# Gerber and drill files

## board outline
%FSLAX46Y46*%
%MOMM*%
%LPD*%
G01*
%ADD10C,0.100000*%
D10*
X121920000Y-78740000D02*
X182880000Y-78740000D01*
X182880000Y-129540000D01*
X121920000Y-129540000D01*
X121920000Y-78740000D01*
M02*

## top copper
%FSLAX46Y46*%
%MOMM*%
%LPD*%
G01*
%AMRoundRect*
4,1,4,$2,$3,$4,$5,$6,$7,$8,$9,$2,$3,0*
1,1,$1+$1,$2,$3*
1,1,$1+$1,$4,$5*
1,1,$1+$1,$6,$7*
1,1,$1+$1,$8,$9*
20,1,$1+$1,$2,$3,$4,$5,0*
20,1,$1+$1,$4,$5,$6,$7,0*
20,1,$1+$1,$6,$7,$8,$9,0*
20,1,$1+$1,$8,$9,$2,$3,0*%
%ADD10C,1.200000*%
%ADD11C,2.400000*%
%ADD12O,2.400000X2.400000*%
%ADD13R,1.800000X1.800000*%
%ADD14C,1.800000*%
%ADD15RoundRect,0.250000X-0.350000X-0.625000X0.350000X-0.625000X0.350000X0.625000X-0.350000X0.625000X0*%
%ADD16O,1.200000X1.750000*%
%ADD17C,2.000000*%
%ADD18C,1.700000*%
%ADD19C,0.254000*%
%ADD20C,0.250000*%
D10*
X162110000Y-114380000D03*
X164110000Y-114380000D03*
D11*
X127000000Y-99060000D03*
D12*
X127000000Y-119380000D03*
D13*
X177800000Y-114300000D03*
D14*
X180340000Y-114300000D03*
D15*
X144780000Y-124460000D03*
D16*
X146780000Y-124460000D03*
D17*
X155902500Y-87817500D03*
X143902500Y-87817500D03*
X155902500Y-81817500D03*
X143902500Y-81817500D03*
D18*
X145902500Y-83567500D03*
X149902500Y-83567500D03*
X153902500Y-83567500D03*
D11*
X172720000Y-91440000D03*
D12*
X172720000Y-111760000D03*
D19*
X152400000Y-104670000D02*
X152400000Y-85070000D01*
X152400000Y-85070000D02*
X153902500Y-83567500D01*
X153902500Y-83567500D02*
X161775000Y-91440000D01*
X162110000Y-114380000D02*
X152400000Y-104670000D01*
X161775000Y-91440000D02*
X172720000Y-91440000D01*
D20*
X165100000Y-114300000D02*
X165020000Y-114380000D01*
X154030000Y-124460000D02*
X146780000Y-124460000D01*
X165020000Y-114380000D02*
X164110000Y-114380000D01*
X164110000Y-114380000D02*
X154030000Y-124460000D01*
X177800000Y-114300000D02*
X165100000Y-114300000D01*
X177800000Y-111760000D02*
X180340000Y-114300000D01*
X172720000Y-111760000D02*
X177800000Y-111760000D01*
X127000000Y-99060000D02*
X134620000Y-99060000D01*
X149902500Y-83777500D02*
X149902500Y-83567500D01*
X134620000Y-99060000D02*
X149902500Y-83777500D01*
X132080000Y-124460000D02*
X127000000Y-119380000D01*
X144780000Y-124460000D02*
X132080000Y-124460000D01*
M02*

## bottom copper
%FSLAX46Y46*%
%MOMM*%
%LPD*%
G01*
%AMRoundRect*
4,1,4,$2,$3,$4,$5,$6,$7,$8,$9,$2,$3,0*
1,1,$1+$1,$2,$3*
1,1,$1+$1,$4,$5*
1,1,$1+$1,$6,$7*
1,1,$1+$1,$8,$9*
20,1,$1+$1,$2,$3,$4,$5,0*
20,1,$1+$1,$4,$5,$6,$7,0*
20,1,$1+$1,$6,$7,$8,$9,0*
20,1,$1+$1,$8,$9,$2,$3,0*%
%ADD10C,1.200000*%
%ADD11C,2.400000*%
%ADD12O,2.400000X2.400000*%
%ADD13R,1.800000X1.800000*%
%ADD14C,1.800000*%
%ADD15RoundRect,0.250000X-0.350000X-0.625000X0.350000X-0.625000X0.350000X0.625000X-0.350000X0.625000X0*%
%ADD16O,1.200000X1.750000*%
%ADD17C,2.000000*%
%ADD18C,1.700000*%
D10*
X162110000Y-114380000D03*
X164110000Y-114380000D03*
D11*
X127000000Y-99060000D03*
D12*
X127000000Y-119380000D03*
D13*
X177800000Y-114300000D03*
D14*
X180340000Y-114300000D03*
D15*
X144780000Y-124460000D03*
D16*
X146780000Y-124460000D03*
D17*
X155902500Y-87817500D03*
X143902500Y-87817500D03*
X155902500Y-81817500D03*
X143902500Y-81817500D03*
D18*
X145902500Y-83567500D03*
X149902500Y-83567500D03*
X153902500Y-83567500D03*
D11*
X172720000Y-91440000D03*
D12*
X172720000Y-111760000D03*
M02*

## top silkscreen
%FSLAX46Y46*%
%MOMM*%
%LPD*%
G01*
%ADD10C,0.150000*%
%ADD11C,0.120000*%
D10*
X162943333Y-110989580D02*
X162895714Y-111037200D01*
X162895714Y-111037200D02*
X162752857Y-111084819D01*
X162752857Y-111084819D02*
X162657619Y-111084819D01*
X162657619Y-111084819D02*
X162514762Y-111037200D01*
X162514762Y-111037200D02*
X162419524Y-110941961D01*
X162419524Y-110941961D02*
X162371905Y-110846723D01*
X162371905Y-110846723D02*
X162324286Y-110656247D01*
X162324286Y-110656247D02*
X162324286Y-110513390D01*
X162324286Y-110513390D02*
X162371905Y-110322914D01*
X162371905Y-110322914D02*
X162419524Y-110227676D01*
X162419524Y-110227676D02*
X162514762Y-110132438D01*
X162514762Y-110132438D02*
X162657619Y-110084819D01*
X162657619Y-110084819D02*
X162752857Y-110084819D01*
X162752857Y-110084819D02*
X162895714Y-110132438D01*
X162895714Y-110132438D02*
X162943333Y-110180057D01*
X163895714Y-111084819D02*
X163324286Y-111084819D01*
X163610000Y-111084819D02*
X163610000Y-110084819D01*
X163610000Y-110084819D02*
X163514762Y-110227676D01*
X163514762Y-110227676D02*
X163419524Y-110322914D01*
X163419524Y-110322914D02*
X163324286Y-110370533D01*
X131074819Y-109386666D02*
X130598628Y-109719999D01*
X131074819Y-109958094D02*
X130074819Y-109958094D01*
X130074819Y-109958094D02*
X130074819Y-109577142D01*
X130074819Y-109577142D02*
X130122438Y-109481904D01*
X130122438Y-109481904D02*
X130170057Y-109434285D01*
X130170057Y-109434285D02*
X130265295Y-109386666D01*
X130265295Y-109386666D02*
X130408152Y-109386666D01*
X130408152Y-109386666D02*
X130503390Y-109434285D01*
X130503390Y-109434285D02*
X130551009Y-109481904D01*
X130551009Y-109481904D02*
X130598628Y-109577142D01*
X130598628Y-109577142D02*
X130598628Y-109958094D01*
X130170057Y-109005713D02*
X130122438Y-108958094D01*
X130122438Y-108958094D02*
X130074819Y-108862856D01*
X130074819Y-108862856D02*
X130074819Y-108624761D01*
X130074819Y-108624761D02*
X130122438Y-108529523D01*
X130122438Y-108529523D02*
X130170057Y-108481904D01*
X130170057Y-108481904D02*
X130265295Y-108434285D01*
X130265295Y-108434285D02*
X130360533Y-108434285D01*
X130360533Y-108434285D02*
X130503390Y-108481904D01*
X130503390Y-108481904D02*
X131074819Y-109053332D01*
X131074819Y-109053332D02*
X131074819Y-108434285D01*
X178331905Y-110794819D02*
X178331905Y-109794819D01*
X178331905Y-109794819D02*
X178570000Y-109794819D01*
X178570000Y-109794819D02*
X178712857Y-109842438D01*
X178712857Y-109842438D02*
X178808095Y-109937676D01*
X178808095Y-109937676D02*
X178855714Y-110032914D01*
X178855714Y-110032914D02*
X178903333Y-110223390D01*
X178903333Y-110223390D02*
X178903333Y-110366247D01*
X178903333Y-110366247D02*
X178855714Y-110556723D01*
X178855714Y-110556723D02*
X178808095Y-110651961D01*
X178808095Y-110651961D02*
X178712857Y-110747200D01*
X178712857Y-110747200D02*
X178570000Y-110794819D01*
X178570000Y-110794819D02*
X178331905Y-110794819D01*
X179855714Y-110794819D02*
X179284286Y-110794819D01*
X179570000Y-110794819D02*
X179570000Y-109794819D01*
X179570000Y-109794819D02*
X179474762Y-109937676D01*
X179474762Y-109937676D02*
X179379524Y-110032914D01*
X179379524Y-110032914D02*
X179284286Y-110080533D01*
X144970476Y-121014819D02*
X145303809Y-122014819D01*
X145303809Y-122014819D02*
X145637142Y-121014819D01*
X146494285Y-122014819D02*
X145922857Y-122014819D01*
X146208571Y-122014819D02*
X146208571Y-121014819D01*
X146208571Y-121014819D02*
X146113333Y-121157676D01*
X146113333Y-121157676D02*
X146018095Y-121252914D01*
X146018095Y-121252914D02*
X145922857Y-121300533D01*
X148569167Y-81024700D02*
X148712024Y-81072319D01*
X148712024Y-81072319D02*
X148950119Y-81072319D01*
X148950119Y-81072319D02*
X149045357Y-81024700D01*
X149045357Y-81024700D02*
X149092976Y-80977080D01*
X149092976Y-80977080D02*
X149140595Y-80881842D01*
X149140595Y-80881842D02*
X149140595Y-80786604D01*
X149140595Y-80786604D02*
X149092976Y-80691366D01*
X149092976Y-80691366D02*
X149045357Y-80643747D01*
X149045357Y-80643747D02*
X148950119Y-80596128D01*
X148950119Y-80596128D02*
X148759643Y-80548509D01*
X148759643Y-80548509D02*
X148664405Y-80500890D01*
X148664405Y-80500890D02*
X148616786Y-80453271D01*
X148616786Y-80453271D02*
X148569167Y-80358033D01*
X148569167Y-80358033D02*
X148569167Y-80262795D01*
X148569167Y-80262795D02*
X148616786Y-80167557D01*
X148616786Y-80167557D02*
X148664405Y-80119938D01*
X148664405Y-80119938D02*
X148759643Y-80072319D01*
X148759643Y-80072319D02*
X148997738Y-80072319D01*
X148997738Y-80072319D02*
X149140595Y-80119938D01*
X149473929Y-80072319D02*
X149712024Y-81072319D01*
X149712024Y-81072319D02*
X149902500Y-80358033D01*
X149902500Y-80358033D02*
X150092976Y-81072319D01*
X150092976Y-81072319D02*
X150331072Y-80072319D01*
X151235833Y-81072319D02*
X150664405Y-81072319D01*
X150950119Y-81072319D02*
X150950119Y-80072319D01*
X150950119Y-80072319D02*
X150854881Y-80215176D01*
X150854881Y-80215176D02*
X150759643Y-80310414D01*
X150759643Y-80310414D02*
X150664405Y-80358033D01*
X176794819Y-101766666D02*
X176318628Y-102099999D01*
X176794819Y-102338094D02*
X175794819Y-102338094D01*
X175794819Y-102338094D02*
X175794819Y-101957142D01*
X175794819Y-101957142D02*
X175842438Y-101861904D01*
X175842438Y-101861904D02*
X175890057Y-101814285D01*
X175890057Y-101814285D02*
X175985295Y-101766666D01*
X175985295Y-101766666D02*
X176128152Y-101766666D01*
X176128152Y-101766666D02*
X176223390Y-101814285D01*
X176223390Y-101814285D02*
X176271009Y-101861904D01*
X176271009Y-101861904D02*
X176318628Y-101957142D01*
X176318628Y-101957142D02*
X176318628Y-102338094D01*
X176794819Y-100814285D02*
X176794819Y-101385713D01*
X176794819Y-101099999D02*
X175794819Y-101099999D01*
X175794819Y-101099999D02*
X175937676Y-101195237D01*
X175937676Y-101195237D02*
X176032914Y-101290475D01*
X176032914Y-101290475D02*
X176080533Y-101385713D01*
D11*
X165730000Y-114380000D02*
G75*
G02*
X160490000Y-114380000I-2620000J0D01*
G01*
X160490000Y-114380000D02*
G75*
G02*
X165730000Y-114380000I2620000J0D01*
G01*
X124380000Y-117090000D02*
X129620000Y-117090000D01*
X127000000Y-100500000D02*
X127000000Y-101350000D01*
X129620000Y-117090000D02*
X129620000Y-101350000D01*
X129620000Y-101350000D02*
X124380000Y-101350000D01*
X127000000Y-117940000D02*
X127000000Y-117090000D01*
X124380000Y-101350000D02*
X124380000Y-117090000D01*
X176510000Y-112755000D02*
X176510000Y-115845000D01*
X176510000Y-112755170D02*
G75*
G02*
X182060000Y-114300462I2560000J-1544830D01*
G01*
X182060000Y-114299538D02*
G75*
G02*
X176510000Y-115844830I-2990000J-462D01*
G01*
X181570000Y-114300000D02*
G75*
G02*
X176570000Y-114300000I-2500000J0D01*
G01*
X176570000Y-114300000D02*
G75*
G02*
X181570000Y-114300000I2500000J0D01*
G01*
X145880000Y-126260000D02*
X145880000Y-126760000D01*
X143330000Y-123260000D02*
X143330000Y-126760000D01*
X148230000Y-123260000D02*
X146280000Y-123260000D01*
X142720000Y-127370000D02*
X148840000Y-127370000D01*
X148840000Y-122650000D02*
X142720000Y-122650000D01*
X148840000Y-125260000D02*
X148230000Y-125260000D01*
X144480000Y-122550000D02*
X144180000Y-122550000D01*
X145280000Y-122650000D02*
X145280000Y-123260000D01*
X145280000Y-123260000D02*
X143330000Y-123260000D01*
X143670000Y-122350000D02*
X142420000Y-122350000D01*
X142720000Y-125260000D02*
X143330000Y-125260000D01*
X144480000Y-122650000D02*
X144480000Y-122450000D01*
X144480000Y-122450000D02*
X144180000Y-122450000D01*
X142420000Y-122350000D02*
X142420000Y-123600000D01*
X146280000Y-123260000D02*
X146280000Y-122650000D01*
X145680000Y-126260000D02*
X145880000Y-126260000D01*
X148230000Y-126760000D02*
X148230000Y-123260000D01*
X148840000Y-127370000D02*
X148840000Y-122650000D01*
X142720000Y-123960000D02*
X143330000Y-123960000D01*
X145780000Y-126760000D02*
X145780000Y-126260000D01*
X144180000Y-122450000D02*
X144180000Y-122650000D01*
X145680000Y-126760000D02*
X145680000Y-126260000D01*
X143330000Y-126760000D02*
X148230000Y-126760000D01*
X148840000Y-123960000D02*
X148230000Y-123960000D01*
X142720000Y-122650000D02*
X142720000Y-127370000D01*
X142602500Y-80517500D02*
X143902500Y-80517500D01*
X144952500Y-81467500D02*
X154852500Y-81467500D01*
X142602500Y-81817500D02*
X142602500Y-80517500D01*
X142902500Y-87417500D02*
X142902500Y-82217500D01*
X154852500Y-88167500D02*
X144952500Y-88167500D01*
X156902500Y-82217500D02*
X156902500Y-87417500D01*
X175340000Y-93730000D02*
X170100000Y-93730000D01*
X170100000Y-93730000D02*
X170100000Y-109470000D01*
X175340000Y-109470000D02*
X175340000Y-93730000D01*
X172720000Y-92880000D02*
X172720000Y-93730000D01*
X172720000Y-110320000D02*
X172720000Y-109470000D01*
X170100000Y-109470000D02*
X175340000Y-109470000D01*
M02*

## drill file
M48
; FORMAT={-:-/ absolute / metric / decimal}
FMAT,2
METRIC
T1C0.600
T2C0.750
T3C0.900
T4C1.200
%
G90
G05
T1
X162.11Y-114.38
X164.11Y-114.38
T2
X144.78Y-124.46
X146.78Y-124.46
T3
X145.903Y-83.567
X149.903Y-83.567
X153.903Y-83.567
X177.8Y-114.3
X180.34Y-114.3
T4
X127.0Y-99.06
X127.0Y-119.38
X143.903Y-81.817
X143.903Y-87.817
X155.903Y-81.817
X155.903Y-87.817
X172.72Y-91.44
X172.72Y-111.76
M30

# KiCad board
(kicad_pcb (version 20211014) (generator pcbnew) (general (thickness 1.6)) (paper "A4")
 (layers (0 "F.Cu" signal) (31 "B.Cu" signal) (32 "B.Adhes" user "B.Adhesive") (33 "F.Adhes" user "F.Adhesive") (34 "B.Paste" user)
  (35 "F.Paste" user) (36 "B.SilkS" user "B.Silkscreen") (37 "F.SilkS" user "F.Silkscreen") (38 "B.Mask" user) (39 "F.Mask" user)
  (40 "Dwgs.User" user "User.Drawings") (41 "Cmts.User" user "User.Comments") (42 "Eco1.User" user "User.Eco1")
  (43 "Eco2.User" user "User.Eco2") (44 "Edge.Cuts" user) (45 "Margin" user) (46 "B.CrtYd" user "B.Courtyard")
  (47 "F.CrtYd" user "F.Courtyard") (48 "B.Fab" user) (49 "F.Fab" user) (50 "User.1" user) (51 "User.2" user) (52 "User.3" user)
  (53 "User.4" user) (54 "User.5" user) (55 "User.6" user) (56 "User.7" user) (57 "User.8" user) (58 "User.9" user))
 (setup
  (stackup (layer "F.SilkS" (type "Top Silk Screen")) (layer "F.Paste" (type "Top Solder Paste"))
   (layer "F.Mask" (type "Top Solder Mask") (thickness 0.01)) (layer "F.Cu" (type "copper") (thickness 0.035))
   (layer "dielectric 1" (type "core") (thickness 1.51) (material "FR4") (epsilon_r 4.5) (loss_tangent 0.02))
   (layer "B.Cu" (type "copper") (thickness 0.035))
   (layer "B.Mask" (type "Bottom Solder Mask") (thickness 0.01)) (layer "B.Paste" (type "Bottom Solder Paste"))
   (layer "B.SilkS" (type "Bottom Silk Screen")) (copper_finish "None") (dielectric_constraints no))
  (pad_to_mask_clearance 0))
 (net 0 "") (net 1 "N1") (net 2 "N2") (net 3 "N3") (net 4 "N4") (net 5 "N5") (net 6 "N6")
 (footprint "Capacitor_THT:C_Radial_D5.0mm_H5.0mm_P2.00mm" (layer "F.Cu") (at 162.11 114.38)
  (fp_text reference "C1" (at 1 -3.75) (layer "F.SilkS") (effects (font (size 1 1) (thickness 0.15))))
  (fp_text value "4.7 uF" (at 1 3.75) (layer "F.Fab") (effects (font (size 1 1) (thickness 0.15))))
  (fp_circle (center 1 0) (end 3.62 0) (layer "F.SilkS") (width 0.12) (fill none))
  (pad "1" thru_hole circle (at 0 0) (size 1.2 1.2) (drill 0.6) (layers *.Cu *.Mask) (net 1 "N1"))
  (pad "2" thru_hole circle (at 2 0) (size 1.2 1.2) (drill 0.6) (layers *.Cu *.Mask) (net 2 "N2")))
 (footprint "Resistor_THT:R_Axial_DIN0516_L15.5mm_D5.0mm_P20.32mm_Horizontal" (layer "F.Cu") (at 127 99.06 -90)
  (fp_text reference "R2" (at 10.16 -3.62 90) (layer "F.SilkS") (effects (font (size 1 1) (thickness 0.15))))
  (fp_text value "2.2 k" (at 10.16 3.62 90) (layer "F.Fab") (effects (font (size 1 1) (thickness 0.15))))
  (fp_line (start 18.03 2.62) (end 18.03 -2.62) (layer "F.SilkS") (width 0.12))
  (fp_line (start 1.44 0) (end 2.29 0) (layer "F.SilkS") (width 0.12))
  (fp_line (start 18.03 -2.62) (end 2.29 -2.62) (layer "F.SilkS") (width 0.12))
  (fp_line (start 2.29 -2.62) (end 2.29 2.62) (layer "F.SilkS") (width 0.12))
  (fp_line (start 18.88 0) (end 18.03 0) (layer "F.SilkS") (width 0.12))
  (fp_line (start 2.29 2.62) (end 18.03 2.62) (layer "F.SilkS") (width 0.12))
  (pad "1" thru_hole circle (at 0 0 270) (size 2.4 2.4) (drill 1.2) (layers *.Cu *.Mask) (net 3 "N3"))
  (pad "2" thru_hole oval (at 20.32 0 270) (size 2.4 2.4) (drill 1.2) (layers *.Cu *.Mask) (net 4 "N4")))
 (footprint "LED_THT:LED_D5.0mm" (layer "F.Cu") (at 177.8 114.3)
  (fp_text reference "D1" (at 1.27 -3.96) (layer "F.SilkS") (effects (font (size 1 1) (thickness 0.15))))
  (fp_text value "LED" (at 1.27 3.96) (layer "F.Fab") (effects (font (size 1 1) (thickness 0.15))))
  (fp_line (start -1.29 -1.545) (end -1.29 1.545) (layer "F.SilkS") (width 0.12))
  (fp_arc (start -1.29 -1.54483) (mid 2.072002 -2.880433) (end 4.26 0.000462) (layer "F.SilkS") (width 0.12))
  (fp_arc (start 4.26 -0.000462) (mid 2.072002 2.880433) (end -1.29 1.54483) (layer "F.SilkS") (width 0.12))
  (fp_circle (center 1.27 0) (end 3.77 0) (layer "F.SilkS") (width 0.12) (fill none))
  (pad "1" thru_hole rect (at 0 0) (size 1.8 1.8) (drill 0.9) (layers *.Cu *.Mask) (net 2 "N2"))
  (pad "2" thru_hole circle (at 2.54 0) (size 1.8 1.8) (drill 0.9) (layers *.Cu *.Mask) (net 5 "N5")))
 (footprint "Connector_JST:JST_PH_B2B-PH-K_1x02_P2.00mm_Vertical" (layer "F.Cu") (at 144.78 124.46)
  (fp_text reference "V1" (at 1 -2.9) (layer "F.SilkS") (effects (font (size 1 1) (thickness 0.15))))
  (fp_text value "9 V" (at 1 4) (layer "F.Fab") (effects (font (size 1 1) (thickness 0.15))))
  (fp_line (start 1.1 1.8) (end 1.1 2.3) (layer "F.SilkS") (width 0.12))
  (fp_line (start -1.45 -1.2) (end -1.45 2.3) (layer "F.SilkS") (width 0.12))
  (fp_line (start 3.45 -1.2) (end 1.5 -1.2) (layer "F.SilkS") (width 0.12))
  (fp_line (start -2.06 2.91) (end 4.06 2.91) (layer "F.SilkS") (width 0.12))
  (fp_line (start 4.06 -1.81) (end -2.06 -1.81) (layer "F.SilkS") (width 0.12))
  (fp_line (start 4.06 0.8) (end 3.45 0.8) (layer "F.SilkS") (width 0.12))
  (fp_line (start -0.3 -1.91) (end -0.6 -1.91) (layer "F.SilkS") (width 0.12))
  (fp_line (start 0.5 -1.81) (end 0.5 -1.2) (layer "F.SilkS") (width 0.12))
  (fp_line (start 0.5 -1.2) (end -1.45 -1.2) (layer "F.SilkS") (width 0.12))
  (fp_line (start -1.11 -2.11) (end -2.36 -2.11) (layer "F.SilkS") (width 0.12))
  (fp_line (start -2.06 0.8) (end -1.45 0.8) (layer "F.SilkS") (width 0.12))
  (fp_line (start -0.3 -1.81) (end -0.3 -2.01) (layer "F.SilkS") (width 0.12))
  (fp_line (start -0.3 -2.01) (end -0.6 -2.01) (layer "F.SilkS") (width 0.12))
  (fp_line (start -2.36 -2.11) (end -2.36 -0.86) (layer "F.SilkS") (width 0.12))
  (fp_line (start 1.5 -1.2) (end 1.5 -1.81) (layer "F.SilkS") (width 0.12))
  (fp_line (start 0.9 1.8) (end 1.1 1.8) (layer "F.SilkS") (width 0.12))
  (fp_line (start 3.45 2.3) (end 3.45 -1.2) (layer "F.SilkS") (width 0.12))
  (fp_line (start 4.06 2.91) (end 4.06 -1.81) (layer "F.SilkS") (width 0.12))
  (fp_line (start -2.06 -0.5) (end -1.45 -0.5) (layer "F.SilkS") (width 0.12))
  (fp_line (start 1 2.3) (end 1 1.8) (layer "F.SilkS") (width 0.12))
  (fp_line (start -0.6 -2.01) (end -0.6 -1.81) (layer "F.SilkS") (width 0.12))
  (fp_line (start 0.9 2.3) (end 0.9 1.8) (layer "F.SilkS") (width 0.12))
  (fp_line (start -1.45 2.3) (end 3.45 2.3) (layer "F.SilkS") (width 0.12))
  (fp_line (start 4.06 -0.5) (end 3.45 -0.5) (layer "F.SilkS") (width 0.12))
  (fp_line (start -2.06 -1.81) (end -2.06 2.91) (layer "F.SilkS") (width 0.12))
  (pad "1" thru_hole roundrect (at 0 0) (size 1.2 1.75) (drill 0.75) (layers *.Cu *.Mask) (roundrect_rratio 0.208333) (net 4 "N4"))
  (pad "2" thru_hole oval (at 2 0) (size 1.2 1.75) (drill 0.75) (layers *.Cu *.Mask) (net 2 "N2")))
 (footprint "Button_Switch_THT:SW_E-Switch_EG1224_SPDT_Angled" (layer "F.Cu") (at 145.9025 83.5675)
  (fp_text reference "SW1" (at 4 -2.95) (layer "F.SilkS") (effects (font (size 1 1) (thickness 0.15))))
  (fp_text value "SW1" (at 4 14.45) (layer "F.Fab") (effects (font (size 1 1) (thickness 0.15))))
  (fp_line (start -3.3 -3.05) (end -2 -3.05) (layer "F.SilkS") (width 0.12))
  (fp_line (start -0.95 -2.1) (end 8.95 -2.1) (layer "F.SilkS") (width 0.12))
  (fp_line (start -3.3 -1.75) (end -3.3 -3.05) (layer "F.SilkS") (width 0.12))
  (fp_line (start -3 3.85) (end -3 -1.35) (layer "F.SilkS") (width 0.12))
  (fp_line (start 8.95 4.6) (end -0.95 4.6) (layer "F.SilkS") (width 0.12))
  (fp_line (start 11 -1.35) (end 11 3.85) (layer "F.SilkS") (width 0.12))
  (pad "" thru_hole circle (at 10 4.25) (size 2 2) (drill 1.2) (layers *.Cu *.Mask))
  (pad "" thru_hole circle (at -2 4.25) (size 2 2) (drill 1.2) (layers *.Cu *.Mask))
  (pad "" thru_hole circle (at 10 -1.75) (size 2 2) (drill 1.2) (layers *.Cu *.Mask))
  (pad "" thru_hole circle (at -2 -1.75) (size 2 2) (drill 1.2) (layers *.Cu *.Mask))
  (pad "1" thru_hole circle (at 0 0) (size 1.7 1.7) (drill 0.9) (layers *.Cu *.Mask) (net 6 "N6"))
  (pad "2" thru_hole circle (at 4 0) (size 1.7 1.7) (drill 0.9) (layers *.Cu *.Mask) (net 3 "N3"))
  (pad "3" thru_hole circle (at 8 0) (size 1.7 1.7) (drill 0.9) (layers *.Cu *.Mask) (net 1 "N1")))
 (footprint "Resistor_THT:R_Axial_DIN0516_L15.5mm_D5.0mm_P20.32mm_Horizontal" (layer "F.Cu") (at 172.72 91.44 -90)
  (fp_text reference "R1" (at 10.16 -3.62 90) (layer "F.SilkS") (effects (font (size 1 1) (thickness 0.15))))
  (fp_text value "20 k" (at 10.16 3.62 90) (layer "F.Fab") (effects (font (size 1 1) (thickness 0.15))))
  (fp_line (start 2.29 -2.62) (end 2.29 2.62) (layer "F.SilkS") (width 0.12))
  (fp_line (start 2.29 2.62) (end 18.03 2.62) (layer "F.SilkS") (width 0.12))
  (fp_line (start 18.03 -2.62) (end 2.29 -2.62) (layer "F.SilkS") (width 0.12))
  (fp_line (start 1.44 0) (end 2.29 0) (layer "F.SilkS") (width 0.12))
  (fp_line (start 18.88 0) (end 18.03 0) (layer "F.SilkS") (width 0.12))
  (fp_line (start 18.03 2.62) (end 18.03 -2.62) (layer "F.SilkS") (width 0.12))
  (pad "1" thru_hole circle (at 0 0 270) (size 2.4 2.4) (drill 1.2) (layers *.Cu *.Mask) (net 1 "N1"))
  (pad "2" thru_hole oval (at 20.32 0 270) (size 2.4 2.4) (drill 1.2) (layers *.Cu *.Mask) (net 5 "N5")))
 (gr_rect (start 182.88 129.54) (end 121.92 78.74) (layer "Edge.Cuts") (width 0.1) (fill none))
 (segment (start 152.4 104.67) (end 152.4 85.07) (width 0.254) (layer "F.Cu") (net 1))
 (segment (start 152.4 85.07) (end 153.9025 83.5675) (width 0.254) (layer "F.Cu") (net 1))
 (segment (start 153.9025 83.5675) (end 161.775 91.44) (width 0.254) (layer "F.Cu") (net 1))
 (segment (start 162.11 114.38) (end 152.4 104.67) (width 0.254) (layer "F.Cu") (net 1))
 (segment (start 161.775 91.44) (end 172.72 91.44) (width 0.254) (layer "F.Cu") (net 1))
 (segment (start 165.1 114.3) (end 165.02 114.38) (width 0.25) (layer "F.Cu") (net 2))
 (segment (start 154.03 124.46) (end 146.78 124.46) (width 0.25) (layer "F.Cu") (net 2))
 (segment (start 165.02 114.38) (end 164.11 114.38) (width 0.25) (layer "F.Cu") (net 2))
 (segment (start 164.11 114.38) (end 154.03 124.46) (width 0.25) (layer "F.Cu") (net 2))
 (segment (start 177.8 114.3) (end 165.1 114.3) (width 0.25) (layer "F.Cu") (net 2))
 (segment (start 177.8 111.76) (end 180.34 114.3) (width 0.25) (layer "F.Cu") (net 5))
 (segment (start 172.72 111.76) (end 177.8 111.76) (width 0.25) (layer "F.Cu") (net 5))
 (segment (start 127 99.06) (end 134.62 99.06) (width 0.25) (layer "F.Cu") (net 3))
 (segment (start 149.9025 83.7775) (end 149.9025 83.5675) (width 0.25) (layer "F.Cu") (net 3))
 (segment (start 134.62 99.06) (end 149.9025 83.7775) (width 0.25) (layer "F.Cu") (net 3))
 (segment (start 132.08 124.46) (end 127 119.38) (width 0.25) (layer "F.Cu") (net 4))
 (segment (start 144.78 124.46) (end 132.08 124.46) (width 0.25) (layer "F.Cu") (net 4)))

